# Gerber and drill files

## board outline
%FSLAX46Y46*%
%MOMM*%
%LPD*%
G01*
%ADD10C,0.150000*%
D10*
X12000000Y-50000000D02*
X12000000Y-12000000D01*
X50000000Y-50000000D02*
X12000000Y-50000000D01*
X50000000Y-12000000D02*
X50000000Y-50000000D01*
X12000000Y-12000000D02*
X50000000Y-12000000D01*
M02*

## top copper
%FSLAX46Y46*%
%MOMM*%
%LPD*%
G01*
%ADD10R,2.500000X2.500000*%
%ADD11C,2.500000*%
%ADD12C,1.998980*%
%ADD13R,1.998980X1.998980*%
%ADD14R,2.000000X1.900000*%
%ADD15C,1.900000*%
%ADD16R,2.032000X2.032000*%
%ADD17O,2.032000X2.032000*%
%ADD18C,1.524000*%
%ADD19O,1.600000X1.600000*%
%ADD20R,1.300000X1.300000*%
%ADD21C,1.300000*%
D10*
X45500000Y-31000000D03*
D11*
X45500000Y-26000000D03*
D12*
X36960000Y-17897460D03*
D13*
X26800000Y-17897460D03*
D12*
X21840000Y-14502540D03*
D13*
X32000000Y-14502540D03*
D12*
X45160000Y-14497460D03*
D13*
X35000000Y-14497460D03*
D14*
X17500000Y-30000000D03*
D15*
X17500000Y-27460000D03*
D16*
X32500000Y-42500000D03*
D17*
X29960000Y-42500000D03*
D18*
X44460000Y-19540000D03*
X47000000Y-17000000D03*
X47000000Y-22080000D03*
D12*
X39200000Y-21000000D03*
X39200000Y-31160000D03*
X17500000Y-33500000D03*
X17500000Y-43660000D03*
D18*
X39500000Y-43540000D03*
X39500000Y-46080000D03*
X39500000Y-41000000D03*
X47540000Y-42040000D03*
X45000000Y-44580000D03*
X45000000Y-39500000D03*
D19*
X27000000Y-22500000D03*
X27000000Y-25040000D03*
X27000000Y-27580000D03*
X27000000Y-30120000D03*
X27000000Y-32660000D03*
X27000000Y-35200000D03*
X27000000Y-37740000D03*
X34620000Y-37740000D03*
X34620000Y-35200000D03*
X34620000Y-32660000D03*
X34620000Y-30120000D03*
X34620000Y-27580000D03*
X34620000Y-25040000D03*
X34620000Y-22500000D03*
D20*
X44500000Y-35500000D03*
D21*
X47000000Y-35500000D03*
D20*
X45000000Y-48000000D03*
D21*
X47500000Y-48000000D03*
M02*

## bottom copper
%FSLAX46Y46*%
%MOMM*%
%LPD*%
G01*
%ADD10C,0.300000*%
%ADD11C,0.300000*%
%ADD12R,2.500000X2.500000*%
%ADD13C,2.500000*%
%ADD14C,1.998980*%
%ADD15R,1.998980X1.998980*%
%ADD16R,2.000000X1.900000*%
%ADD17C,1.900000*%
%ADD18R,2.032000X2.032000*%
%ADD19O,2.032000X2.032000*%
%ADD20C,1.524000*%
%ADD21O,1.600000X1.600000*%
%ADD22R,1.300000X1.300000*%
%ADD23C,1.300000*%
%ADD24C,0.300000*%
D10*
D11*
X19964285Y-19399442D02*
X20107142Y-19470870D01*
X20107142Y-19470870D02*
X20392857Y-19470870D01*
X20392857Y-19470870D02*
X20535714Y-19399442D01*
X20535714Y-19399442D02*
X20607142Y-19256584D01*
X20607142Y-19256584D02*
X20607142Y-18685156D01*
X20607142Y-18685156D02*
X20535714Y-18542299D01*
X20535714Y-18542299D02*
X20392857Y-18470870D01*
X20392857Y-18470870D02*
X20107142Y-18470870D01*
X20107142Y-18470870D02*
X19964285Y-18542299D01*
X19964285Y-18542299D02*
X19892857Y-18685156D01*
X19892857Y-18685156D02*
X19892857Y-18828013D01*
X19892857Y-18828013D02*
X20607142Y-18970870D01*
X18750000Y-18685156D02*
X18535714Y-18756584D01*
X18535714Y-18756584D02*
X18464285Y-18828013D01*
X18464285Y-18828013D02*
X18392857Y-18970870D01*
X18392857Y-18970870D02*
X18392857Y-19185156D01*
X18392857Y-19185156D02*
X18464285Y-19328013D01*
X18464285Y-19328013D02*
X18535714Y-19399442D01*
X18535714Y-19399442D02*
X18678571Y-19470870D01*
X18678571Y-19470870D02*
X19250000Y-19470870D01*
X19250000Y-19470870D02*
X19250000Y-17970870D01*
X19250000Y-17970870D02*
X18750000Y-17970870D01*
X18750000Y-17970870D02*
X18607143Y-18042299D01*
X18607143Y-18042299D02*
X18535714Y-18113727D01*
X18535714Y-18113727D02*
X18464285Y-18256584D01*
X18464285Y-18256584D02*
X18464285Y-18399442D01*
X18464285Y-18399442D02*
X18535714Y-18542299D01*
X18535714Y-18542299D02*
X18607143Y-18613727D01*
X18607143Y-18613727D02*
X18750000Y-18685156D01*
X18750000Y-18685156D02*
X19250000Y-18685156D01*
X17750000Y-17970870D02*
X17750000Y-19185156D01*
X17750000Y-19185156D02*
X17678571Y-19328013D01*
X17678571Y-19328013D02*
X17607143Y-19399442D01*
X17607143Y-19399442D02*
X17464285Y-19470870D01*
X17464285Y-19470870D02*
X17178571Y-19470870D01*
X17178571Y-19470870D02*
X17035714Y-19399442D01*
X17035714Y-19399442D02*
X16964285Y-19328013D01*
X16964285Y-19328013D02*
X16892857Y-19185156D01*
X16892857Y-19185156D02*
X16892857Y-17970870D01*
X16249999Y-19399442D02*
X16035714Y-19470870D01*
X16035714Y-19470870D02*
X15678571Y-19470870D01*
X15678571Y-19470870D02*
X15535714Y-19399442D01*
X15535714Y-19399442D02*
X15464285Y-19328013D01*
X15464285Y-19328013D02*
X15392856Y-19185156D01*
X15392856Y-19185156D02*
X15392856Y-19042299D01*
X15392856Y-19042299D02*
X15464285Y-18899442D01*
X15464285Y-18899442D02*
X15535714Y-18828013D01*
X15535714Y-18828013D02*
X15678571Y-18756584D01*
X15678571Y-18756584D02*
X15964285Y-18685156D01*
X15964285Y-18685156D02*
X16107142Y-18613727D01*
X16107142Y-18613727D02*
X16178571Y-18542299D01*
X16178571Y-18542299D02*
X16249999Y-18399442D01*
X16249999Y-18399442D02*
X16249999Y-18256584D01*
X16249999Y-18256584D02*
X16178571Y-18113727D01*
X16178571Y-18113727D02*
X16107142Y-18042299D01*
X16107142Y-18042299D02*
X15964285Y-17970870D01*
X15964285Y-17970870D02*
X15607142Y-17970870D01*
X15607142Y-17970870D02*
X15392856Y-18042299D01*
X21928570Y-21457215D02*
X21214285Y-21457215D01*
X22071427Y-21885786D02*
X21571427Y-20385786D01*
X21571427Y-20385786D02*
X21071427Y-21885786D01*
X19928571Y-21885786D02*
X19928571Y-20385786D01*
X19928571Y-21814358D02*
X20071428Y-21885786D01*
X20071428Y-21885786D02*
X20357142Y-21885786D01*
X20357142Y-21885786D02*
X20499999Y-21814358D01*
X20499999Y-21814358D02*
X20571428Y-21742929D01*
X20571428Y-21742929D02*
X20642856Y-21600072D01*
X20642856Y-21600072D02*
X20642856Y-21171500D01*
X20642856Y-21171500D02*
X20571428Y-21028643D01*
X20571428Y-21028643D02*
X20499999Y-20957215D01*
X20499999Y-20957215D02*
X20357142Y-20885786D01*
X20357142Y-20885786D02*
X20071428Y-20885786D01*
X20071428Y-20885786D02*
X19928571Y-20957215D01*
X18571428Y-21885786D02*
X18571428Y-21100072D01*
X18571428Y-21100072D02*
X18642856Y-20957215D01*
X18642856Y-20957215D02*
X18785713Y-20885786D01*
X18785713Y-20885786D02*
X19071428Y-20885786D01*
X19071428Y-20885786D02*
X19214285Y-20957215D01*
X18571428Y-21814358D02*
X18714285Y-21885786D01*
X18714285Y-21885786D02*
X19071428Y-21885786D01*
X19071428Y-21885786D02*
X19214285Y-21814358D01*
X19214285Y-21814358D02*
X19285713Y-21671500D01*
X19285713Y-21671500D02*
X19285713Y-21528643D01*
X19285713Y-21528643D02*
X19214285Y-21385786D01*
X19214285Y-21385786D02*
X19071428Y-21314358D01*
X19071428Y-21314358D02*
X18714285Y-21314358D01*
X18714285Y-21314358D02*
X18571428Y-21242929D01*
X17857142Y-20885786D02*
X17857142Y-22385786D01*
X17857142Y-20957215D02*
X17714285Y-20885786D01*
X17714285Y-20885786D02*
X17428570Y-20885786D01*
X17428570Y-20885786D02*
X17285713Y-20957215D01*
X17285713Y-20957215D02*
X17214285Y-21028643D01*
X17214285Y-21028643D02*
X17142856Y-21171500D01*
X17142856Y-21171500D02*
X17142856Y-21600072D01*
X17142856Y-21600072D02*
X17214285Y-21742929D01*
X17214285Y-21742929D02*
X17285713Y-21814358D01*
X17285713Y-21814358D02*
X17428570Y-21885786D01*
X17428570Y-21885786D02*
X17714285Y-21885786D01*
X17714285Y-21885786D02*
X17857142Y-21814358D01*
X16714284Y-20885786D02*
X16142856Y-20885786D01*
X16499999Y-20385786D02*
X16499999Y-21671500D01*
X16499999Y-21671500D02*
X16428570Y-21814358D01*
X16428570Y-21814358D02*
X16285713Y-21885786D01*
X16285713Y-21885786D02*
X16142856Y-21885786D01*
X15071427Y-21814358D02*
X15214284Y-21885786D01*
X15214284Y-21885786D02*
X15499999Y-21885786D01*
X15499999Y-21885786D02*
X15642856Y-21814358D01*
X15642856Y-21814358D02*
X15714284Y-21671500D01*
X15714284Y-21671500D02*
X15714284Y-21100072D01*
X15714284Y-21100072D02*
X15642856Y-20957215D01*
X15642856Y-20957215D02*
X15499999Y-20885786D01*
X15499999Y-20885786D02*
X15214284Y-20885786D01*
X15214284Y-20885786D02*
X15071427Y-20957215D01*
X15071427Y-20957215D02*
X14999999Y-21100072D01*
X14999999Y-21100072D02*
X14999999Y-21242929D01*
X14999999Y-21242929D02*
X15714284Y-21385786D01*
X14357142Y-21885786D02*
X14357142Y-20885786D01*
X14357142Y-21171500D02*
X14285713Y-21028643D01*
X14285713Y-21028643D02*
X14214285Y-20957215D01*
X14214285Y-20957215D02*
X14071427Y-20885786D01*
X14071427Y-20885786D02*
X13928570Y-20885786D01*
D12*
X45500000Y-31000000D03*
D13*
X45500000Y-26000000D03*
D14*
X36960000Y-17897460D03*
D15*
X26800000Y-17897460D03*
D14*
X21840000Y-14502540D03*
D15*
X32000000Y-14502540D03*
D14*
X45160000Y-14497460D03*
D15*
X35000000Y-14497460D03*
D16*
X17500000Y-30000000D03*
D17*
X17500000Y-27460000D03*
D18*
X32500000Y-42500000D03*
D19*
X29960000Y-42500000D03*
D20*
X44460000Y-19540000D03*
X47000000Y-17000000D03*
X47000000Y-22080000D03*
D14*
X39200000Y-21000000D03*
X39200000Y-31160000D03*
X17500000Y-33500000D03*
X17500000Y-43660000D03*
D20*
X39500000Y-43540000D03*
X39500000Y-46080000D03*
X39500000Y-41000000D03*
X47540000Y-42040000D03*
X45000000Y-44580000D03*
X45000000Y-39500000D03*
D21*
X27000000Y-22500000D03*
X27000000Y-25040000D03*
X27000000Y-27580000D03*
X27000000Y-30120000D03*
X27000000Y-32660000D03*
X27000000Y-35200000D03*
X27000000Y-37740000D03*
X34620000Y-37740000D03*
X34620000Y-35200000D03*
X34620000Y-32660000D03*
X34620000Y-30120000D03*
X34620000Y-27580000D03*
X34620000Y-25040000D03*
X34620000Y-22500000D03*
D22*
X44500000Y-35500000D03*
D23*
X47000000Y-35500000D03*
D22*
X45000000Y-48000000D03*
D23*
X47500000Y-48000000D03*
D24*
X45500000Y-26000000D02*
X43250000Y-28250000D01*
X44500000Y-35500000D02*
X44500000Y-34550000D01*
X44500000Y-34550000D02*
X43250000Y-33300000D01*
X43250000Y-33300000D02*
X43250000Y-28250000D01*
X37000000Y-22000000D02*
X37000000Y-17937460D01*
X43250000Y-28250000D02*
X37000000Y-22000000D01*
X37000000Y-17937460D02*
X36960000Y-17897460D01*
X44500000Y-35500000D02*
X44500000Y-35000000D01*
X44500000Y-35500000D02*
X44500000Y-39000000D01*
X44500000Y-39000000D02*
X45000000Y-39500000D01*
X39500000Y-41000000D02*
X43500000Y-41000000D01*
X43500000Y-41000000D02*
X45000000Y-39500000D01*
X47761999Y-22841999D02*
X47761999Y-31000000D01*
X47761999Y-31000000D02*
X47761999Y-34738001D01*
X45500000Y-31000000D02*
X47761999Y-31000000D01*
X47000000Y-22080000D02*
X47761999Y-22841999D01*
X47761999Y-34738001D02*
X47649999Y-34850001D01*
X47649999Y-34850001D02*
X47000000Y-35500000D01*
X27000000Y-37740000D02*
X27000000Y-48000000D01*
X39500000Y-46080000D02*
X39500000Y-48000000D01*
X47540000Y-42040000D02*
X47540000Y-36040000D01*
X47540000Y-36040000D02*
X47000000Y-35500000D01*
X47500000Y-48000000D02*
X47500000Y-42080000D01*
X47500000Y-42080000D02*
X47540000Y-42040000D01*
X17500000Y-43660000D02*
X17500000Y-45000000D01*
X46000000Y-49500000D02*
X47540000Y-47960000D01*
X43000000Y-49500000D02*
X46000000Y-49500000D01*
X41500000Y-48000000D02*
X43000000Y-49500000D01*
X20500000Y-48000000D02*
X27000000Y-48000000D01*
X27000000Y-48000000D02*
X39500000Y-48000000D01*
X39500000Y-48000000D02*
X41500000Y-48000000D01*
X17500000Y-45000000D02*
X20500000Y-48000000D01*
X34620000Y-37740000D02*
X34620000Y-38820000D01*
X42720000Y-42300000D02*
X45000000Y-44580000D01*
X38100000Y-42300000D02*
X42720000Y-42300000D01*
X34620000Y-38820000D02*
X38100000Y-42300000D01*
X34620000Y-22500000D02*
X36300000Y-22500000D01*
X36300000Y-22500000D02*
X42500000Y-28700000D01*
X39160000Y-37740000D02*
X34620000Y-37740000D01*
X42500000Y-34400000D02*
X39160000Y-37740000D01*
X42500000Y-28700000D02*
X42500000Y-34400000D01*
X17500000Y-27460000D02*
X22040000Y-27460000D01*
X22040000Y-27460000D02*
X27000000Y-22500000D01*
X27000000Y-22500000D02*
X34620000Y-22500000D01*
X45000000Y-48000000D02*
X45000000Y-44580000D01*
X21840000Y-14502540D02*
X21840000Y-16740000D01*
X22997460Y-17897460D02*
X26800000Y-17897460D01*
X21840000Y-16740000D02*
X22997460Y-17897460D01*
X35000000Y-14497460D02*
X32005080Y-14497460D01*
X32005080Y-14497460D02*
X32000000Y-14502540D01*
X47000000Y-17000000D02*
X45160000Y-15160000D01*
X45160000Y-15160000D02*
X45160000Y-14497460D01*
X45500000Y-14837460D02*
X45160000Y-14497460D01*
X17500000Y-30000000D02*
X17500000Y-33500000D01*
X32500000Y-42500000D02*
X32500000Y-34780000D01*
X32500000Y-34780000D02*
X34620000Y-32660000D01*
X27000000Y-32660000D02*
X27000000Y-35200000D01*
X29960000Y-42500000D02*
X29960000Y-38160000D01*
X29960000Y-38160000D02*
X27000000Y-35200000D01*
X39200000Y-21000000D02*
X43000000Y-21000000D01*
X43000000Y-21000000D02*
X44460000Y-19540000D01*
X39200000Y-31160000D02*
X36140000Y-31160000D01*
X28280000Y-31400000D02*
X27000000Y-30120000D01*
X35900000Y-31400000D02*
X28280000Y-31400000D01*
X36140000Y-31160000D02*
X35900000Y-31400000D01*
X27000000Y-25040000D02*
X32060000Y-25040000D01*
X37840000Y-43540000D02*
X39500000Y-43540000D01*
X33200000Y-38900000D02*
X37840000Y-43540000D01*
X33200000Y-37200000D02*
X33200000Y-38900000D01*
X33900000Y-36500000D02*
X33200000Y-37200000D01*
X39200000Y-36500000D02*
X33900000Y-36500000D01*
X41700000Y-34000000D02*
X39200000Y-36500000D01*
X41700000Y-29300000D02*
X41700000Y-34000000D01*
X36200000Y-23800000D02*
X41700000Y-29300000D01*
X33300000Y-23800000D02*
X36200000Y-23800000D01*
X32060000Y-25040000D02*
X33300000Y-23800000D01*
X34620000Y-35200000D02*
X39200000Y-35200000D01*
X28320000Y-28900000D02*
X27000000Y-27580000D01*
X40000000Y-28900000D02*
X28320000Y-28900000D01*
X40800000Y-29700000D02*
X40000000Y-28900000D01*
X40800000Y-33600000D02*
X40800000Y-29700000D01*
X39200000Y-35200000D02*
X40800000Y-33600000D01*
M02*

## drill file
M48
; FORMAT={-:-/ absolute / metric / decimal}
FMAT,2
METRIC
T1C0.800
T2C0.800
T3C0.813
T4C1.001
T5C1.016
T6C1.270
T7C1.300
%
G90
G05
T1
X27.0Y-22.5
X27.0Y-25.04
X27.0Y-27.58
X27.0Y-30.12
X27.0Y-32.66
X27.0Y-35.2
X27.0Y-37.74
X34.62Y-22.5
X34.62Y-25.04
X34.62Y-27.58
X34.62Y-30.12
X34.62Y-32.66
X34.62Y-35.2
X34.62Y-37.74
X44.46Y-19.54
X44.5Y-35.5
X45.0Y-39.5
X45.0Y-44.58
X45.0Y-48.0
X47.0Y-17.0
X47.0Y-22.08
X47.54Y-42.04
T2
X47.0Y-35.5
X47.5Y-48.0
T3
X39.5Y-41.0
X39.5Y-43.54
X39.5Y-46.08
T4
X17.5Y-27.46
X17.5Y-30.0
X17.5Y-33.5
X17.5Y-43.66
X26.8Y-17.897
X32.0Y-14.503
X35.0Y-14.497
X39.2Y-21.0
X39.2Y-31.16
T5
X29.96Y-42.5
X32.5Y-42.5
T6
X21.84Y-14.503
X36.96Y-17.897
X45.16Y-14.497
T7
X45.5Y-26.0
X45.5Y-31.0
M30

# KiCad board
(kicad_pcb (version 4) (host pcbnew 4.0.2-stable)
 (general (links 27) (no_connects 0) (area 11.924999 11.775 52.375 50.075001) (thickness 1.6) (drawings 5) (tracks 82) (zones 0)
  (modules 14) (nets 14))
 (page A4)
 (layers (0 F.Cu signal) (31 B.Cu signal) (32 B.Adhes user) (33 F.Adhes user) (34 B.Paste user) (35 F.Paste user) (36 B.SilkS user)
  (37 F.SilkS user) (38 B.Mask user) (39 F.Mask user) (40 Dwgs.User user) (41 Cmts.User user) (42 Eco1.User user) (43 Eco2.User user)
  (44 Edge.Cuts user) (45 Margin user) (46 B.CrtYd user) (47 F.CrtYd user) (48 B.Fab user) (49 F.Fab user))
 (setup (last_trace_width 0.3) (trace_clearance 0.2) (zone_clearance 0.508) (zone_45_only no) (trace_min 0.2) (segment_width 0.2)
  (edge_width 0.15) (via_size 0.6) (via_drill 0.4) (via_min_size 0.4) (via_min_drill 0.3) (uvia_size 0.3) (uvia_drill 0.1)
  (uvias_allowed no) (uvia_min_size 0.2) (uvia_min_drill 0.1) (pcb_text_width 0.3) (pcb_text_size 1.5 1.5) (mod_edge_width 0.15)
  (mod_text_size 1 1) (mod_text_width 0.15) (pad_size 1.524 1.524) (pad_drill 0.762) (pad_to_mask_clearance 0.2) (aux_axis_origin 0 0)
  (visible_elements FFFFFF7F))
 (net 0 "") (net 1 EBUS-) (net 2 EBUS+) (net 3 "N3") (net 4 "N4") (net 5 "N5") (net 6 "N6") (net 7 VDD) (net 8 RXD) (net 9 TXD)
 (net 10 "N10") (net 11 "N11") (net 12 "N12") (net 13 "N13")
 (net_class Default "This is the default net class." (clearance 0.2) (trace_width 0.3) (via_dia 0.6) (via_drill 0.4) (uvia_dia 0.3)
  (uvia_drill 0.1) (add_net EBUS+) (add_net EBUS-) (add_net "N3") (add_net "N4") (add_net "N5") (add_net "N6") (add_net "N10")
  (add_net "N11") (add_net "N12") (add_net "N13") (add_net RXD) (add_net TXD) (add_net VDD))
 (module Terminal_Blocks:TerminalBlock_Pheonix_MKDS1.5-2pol (layer F.Cu) (at 45.5 31 90)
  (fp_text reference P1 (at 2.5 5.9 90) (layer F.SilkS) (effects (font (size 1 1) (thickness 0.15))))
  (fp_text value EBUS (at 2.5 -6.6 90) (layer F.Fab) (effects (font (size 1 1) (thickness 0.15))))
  (pad 1 thru_hole rect (at 0 0 90) (size 2.5 2.5) (drill 1.3) (layers *.Cu *.Mask F.SilkS) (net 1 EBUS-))
  (pad 2 thru_hole circle (at 5 0 90) (size 2.5 2.5) (drill 1.3) (layers *.Cu *.Mask F.SilkS) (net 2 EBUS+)))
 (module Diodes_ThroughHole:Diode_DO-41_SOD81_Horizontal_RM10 (layer F.Cu) (at 26.8 17.9)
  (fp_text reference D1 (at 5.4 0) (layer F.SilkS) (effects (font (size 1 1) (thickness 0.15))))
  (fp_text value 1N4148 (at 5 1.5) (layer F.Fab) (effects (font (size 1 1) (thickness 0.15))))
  (pad 2 thru_hole circle (at 10.16 -0.00254 180) (size 1.99898 1.99898) (drill 1.27) (layers *.Cu *.Mask F.SilkS) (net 2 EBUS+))
  (pad 1 thru_hole rect (at 0 -0.00254 180) (size 1.99898 1.99898) (drill 1.00076) (layers *.Cu *.Mask F.SilkS) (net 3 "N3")))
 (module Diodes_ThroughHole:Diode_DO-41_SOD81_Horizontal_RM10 (layer F.Cu) (at 32 14.5 180)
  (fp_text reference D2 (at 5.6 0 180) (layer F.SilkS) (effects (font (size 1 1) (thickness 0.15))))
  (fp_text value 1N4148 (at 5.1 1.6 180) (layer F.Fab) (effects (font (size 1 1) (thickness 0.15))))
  (pad 2 thru_hole circle (at 10.16 -0.00254) (size 1.99898 1.99898) (drill 1.27) (layers *.Cu *.Mask F.SilkS) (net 3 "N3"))
  (pad 1 thru_hole rect (at 0 -0.00254) (size 1.99898 1.99898) (drill 1.00076) (layers *.Cu *.Mask F.SilkS) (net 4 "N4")))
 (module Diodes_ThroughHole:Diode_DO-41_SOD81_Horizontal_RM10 (layer F.Cu) (at 35 14.5)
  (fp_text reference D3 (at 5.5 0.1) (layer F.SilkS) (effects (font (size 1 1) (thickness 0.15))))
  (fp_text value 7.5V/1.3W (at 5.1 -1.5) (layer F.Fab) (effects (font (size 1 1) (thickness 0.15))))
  (pad 2 thru_hole circle (at 10.16 -0.00254 180) (size 1.99898 1.99898) (drill 1.27) (layers *.Cu *.Mask F.SilkS) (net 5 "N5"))
  (pad 1 thru_hole rect (at 0 -0.00254 180) (size 1.99898 1.99898) (drill 1.00076) (layers *.Cu *.Mask F.SilkS) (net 4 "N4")))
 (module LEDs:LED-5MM (layer F.Cu) (at 17.5 30 90)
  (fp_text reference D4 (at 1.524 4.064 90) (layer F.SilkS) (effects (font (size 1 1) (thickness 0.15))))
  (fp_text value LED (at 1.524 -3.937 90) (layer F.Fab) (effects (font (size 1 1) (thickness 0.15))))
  (pad 1 thru_hole rect (at 0 0 180) (size 2 1.9) (drill 1.00076) (layers *.Cu *.Mask F.SilkS) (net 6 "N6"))
  (pad 2 thru_hole circle (at 2.54 0 90) (size 1.9 1.9) (drill 1.00076) (layers *.Cu *.Mask F.SilkS) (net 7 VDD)))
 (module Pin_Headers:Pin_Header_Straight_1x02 (layer F.Cu) (at 32.5 42.5 270)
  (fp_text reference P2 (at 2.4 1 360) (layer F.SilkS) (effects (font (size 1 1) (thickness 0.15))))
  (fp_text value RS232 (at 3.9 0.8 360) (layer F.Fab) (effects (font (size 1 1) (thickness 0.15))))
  (pad 1 thru_hole rect (at 0 0 270) (size 2.032 2.032) (drill 1.016) (layers *.Cu *.Mask F.SilkS) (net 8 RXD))
  (pad 2 thru_hole oval (at 0 2.54 270) (size 2.032 2.032) (drill 1.016) (layers *.Cu *.Mask F.SilkS) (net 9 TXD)))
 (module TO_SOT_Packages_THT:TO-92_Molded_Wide (layer F.Cu) (at 47 22.08 90)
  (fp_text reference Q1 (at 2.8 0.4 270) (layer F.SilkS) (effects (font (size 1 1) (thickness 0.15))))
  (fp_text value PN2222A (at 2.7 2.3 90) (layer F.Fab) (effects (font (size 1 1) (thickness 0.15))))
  (pad 2 thru_hole circle (at 2.54 -2.54 180) (size 1.524 1.524) (drill 0.8) (layers *.Cu *.Mask F.SilkS) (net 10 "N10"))
  (pad 3 thru_hole circle (at 5.08 0 180) (size 1.524 1.524) (drill 0.8) (layers *.Cu *.Mask F.SilkS) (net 5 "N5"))
  (pad 1 thru_hole circle (at 0 0 180) (size 1.524 1.524) (drill 0.8) (layers *.Cu *.Mask F.SilkS) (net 1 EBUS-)))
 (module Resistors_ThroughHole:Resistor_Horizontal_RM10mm (layer F.Cu) (at 39.2 21 270)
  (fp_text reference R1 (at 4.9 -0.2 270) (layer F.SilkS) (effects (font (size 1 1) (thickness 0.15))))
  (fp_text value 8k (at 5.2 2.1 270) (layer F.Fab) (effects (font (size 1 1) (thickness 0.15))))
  (pad 1 thru_hole circle (at 0 0 270) (size 1.99898 1.99898) (drill 1.00076) (layers *.Cu *.SilkS *.Mask) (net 10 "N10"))
  (pad 2 thru_hole circle (at 10.16 0 270) (size 1.99898 1.99898) (drill 1.00076) (layers *.Cu *.SilkS *.Mask) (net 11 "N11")))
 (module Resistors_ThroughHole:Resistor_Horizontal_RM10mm (layer F.Cu) (at 17.5 33.5 270)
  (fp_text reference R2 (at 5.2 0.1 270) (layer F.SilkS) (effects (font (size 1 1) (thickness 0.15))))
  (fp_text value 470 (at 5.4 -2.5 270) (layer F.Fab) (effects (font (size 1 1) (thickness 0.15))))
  (pad 1 thru_hole circle (at 0 0 270) (size 1.99898 1.99898) (drill 1.00076) (layers *.Cu *.SilkS *.Mask) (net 6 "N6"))
  (pad 2 thru_hole circle (at 10.16 0 270) (size 1.99898 1.99898) (drill 1.00076) (layers *.Cu *.SilkS *.Mask) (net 1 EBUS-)))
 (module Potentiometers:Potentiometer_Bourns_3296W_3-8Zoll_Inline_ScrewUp (layer F.Cu) (at 39.5 41 180)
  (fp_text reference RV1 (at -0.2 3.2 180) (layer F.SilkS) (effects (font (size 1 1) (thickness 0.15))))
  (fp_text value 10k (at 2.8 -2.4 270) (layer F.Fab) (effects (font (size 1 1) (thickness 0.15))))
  (pad 2 thru_hole circle (at 0 -2.54 180) (size 1.524 1.524) (drill 0.8128) (layers *.Cu *.Mask F.SilkS) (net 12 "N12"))
  (pad 3 thru_hole circle (at 0 -5.08 180) (size 1.524 1.524) (drill 0.8128) (layers *.Cu *.Mask F.SilkS) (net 1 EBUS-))
  (pad 1 thru_hole circle (at 0 0 180) (size 1.524 1.524) (drill 0.8128) (layers *.Cu *.Mask F.SilkS) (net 2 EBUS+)))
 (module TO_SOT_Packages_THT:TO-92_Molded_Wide (layer F.Cu) (at 45 39.5 270)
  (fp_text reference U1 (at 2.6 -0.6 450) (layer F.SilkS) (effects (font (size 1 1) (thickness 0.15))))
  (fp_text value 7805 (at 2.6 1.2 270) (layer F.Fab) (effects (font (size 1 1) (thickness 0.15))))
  (pad 2 thru_hole circle (at 2.54 -2.54) (size 1.524 1.524) (drill 0.8) (layers *.Cu *.Mask F.SilkS) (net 1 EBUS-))
  (pad 3 thru_hole circle (at 5.08 0) (size 1.524 1.524) (drill 0.8) (layers *.Cu *.Mask F.SilkS) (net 7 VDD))
  (pad 1 thru_hole circle (at 0 0) (size 1.524 1.524) (drill 0.8) (layers *.Cu *.Mask F.SilkS) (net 2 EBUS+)))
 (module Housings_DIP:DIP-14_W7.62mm (layer F.Cu) (at 27 22.5)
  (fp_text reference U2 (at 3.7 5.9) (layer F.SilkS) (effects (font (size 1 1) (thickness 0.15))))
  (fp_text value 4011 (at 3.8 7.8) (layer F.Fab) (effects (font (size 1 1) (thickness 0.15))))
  (pad 1 thru_hole oval (at 0 0) (size 1.6 1.6) (drill 0.8) (layers *.Cu *.Mask F.SilkS) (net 7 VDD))
  (pad 2 thru_hole oval (at 0 2.54) (size 1.6 1.6) (drill 0.8) (layers *.Cu *.Mask F.SilkS) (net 12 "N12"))
  (pad 3 thru_hole oval (at 0 5.08) (size 1.6 1.6) (drill 0.8) (layers *.Cu *.Mask F.SilkS) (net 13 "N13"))
  (pad 4 thru_hole oval (at 0 7.62) (size 1.6 1.6) (drill 0.8) (layers *.Cu *.Mask F.SilkS) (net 11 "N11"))
  (pad 5 thru_hole oval (at 0 10.16) (size 1.6 1.6) (drill 0.8) (layers *.Cu *.Mask F.SilkS) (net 9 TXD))
  (pad 6 thru_hole oval (at 0 12.7) (size 1.6 1.6) (drill 0.8) (layers *.Cu *.Mask F.SilkS) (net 9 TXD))
  (pad 7 thru_hole oval (at 0 15.24) (size 1.6 1.6) (drill 0.8) (layers *.Cu *.Mask F.SilkS) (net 1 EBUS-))
  (pad 8 thru_hole oval (at 7.62 15.24) (size 1.6 1.6) (drill 0.8) (layers *.Cu *.Mask F.SilkS) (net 7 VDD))
  (pad 9 thru_hole oval (at 7.62 12.7) (size 1.6 1.6) (drill 0.8) (layers *.Cu *.Mask F.SilkS) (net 13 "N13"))
  (pad 10 thru_hole oval (at 7.62 10.16) (size 1.6 1.6) (drill 0.8) (layers *.Cu *.Mask F.SilkS) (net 8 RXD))
  (pad 11 thru_hole oval (at 7.62 7.62) (size 1.6 1.6) (drill 0.8) (layers *.Cu *.Mask F.SilkS))
  (pad 12 thru_hole oval (at 7.62 5.08) (size 1.6 1.6) (drill 0.8) (layers *.Cu *.Mask F.SilkS))
  (pad 13 thru_hole oval (at 7.62 2.54) (size 1.6 1.6) (drill 0.8) (layers *.Cu *.Mask F.SilkS))
  (pad 14 thru_hole oval (at 7.62 0) (size 1.6 1.6) (drill 0.8) (layers *.Cu *.Mask F.SilkS) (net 7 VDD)))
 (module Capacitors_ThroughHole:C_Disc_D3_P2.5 (layer F.Cu) (at 44.5 35.5)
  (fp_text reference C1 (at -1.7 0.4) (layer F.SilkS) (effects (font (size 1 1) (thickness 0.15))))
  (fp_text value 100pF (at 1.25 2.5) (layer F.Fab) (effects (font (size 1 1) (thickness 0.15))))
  (pad 1 thru_hole rect (at 0 0) (size 1.3 1.3) (drill 0.8) (layers *.Cu *.Mask F.SilkS) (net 2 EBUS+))
  (pad 2 thru_hole circle (at 2.5 0) (size 1.3 1.3) (drill 0.8001) (layers *.Cu *.Mask F.SilkS) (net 1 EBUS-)))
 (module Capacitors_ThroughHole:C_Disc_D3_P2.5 (layer F.Cu) (at 45 48)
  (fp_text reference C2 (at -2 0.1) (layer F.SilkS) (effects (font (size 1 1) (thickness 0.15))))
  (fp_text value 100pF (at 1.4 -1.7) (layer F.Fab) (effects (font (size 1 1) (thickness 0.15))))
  (pad 1 thru_hole rect (at 0 0) (size 1.3 1.3) (drill 0.8) (layers *.Cu *.Mask F.SilkS) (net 7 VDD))
  (pad 2 thru_hole circle (at 2.5 0) (size 1.3 1.3) (drill 0.8001) (layers *.Cu *.Mask F.SilkS) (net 1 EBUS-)))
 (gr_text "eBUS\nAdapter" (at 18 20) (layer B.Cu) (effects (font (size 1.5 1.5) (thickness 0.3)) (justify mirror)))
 (gr_line (start 12 50) (end 12 12) (angle 90) (layer Edge.Cuts) (width 0.15))
 (gr_line (start 50 50) (end 12 50) (angle 90) (layer Edge.Cuts) (width 0.15))
 (gr_line (start 50 12) (end 50 50) (angle 90) (layer Edge.Cuts) (width 0.15))
 (gr_line (start 12 12) (end 50 12) (angle 90) (layer Edge.Cuts) (width 0.15))
 (segment (start 45.5 26) (end 43.25 28.25) (width 0.3) (layer B.Cu) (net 2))
 (segment (start 44.5 35.5) (end 44.5 34.55) (width 0.3) (layer B.Cu) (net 2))
 (segment (start 44.5 34.55) (end 43.25 33.3) (width 0.3) (layer B.Cu) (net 2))
 (segment (start 43.25 33.3) (end 43.25 28.25) (width 0.3) (layer B.Cu) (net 2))
 (segment (start 37 22) (end 37 17.93746) (width 0.3) (layer B.Cu) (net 2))
 (segment (start 43.25 28.25) (end 37 22) (width 0.3) (layer B.Cu) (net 2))
 (segment (start 37 17.93746) (end 36.96 17.89746) (width 0.3) (layer B.Cu) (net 2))
 (segment (start 44.5 35.5) (end 44.5 35) (width 0.3) (layer B.Cu) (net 2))
 (segment (start 44.5 35.5) (end 44.5 39) (width 0.3) (layer B.Cu) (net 2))
 (segment (start 44.5 39) (end 45 39.5) (width 0.3) (layer B.Cu) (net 2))
 (segment (start 39.5 41) (end 43.5 41) (width 0.3) (layer B.Cu) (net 2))
 (segment (start 43.5 41) (end 45 39.5) (width 0.3) (layer B.Cu) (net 2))
 (segment (start 47.761999 22.841999) (end 47.761999 31) (width 0.3) (layer B.Cu) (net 1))
 (segment (start 47.761999 31) (end 47.761999 34.738001) (width 0.3) (layer B.Cu) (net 1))
 (segment (start 45.5 31) (end 47.761999 31) (width 0.3) (layer B.Cu) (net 1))
 (segment (start 47 22.08) (end 47.761999 22.841999) (width 0.3) (layer B.Cu) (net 1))
 (segment (start 47.761999 34.738001) (end 47.649999 34.850001) (width 0.3) (layer B.Cu) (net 1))
 (segment (start 47.649999 34.850001) (end 47 35.5) (width 0.3) (layer B.Cu) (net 1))
 (segment (start 27 37.74) (end 27 48) (width 0.3) (layer B.Cu) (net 1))
 (segment (start 39.5 46.08) (end 39.5 48) (width 0.3) (layer B.Cu) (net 1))
 (segment (start 47.54 42.04) (end 47.54 36.04) (width 0.3) (layer B.Cu) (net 1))
 (segment (start 47.54 36.04) (end 47 35.5) (width 0.3) (layer B.Cu) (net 1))
 (segment (start 47.5 48) (end 47.5 42.08) (width 0.3) (layer B.Cu) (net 1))
 (segment (start 47.5 42.08) (end 47.54 42.04) (width 0.3) (layer B.Cu) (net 1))
 (segment (start 17.5 43.66) (end 17.5 45) (width 0.3) (layer B.Cu) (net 1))
 (segment (start 46 49.5) (end 47.54 47.96) (width 0.3) (layer B.Cu) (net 1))
 (segment (start 43 49.5) (end 46 49.5) (width 0.3) (layer B.Cu) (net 1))
 (segment (start 41.5 48) (end 43 49.5) (width 0.3) (layer B.Cu) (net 1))
 (segment (start 20.5 48) (end 27 48) (width 0.3) (layer B.Cu) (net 1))
 (segment (start 27 48) (end 39.5 48) (width 0.3) (layer B.Cu) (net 1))
 (segment (start 39.5 48) (end 41.5 48) (width 0.3) (layer B.Cu) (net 1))
 (segment (start 17.5 45) (end 20.5 48) (width 0.3) (layer B.Cu) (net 1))
 (segment (start 34.62 37.74) (end 34.62 38.82) (width 0.3) (layer B.Cu) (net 7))
 (segment (start 42.72 42.3) (end 45 44.58) (width 0.3) (layer B.Cu) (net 7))
 (segment (start 38.1 42.3) (end 42.72 42.3) (width 0.3) (layer B.Cu) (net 7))
 (segment (start 34.62 38.82) (end 38.1 42.3) (width 0.3) (layer B.Cu) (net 7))
 (segment (start 34.62 22.5) (end 36.3 22.5) (width 0.3) (layer B.Cu) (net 7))
 (segment (start 36.3 22.5) (end 42.5 28.7) (width 0.3) (layer B.Cu) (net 7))
 (segment (start 39.16 37.74) (end 34.62 37.74) (width 0.3) (layer B.Cu) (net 7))
 (segment (start 42.5 34.4) (end 39.16 37.74) (width 0.3) (layer B.Cu) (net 7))
 (segment (start 42.5 28.7) (end 42.5 34.4) (width 0.3) (layer B.Cu) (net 7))
 (segment (start 17.5 27.46) (end 22.04 27.46) (width 0.3) (layer B.Cu) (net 7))
 (segment (start 22.04 27.46) (end 27 22.5) (width 0.3) (layer B.Cu) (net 7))
 (segment (start 27 22.5) (end 34.62 22.5) (width 0.3) (layer B.Cu) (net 7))
 (segment (start 45 48) (end 45 44.58) (width 0.3) (layer B.Cu) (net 7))
 (segment (start 21.84 14.50254) (end 21.84 16.74) (width 0.3) (layer B.Cu) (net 3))
 (segment (start 22.99746 17.89746) (end 26.8 17.89746) (width 0.3) (layer B.Cu) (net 3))
 (segment (start 21.84 16.74) (end 22.99746 17.89746) (width 0.3) (layer B.Cu) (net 3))
 (segment (start 35 14.49746) (end 32.00508 14.49746) (width 0.3) (layer B.Cu) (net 4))
 (segment (start 32.00508 14.49746) (end 32 14.50254) (width 0.3) (layer B.Cu) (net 4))
 (segment (start 47 17) (end 45.16 15.16) (width 0.3) (layer B.Cu) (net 5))
 (segment (start 45.16 15.16) (end 45.16 14.49746) (width 0.3) (layer B.Cu) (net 5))
 (segment (start 45.5 14.83746) (end 45.16 14.49746) (width 0.3) (layer B.Cu) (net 5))
 (segment (start 17.5 30) (end 17.5 33.5) (width 0.3) (layer B.Cu) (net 6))
 (segment (start 32.5 42.5) (end 32.5 34.78) (width 0.3) (layer B.Cu) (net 8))
 (segment (start 32.5 34.78) (end 34.62 32.66) (width 0.3) (layer B.Cu) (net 8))
 (segment (start 27 32.66) (end 27 35.2) (width 0.3) (layer B.Cu) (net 9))
 (segment (start 29.96 42.5) (end 29.96 38.16) (width 0.3) (layer B.Cu) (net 9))
 (segment (start 29.96 38.16) (end 27 35.2) (width 0.3) (layer B.Cu) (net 9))
 (segment (start 39.2 21) (end 43 21) (width 0.3) (layer B.Cu) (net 10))
 (segment (start 43 21) (end 44.46 19.54) (width 0.3) (layer B.Cu) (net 10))
 (segment (start 39.2 31.16) (end 36.14 31.16) (width 0.3) (layer B.Cu) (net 11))
 (segment (start 28.28 31.4) (end 27 30.12) (width 0.3) (layer B.Cu) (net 11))
 (segment (start 35.9 31.4) (end 28.28 31.4) (width 0.3) (layer B.Cu) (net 11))
 (segment (start 36.14 31.16) (end 35.9 31.4) (width 0.3) (layer B.Cu) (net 11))
 (segment (start 27 25.04) (end 32.06 25.04) (width 0.3) (layer B.Cu) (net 12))
 (segment (start 37.84 43.54) (end 39.5 43.54) (width 0.3) (layer B.Cu) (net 12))
 (segment (start 33.2 38.9) (end 37.84 43.54) (width 0.3) (layer B.Cu) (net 12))
 (segment (start 33.2 37.2) (end 33.2 38.9) (width 0.3) (layer B.Cu) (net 12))
 (segment (start 33.9 36.5) (end 33.2 37.2) (width 0.3) (layer B.Cu) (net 12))
 (segment (start 39.2 36.5) (end 33.9 36.5) (width 0.3) (layer B.Cu) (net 12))
 (segment (start 41.7 34) (end 39.2 36.5) (width 0.3) (layer B.Cu) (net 12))
 (segment (start 41.7 29.3) (end 41.7 34) (width 0.3) (layer B.Cu) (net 12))
 (segment (start 36.2 23.8) (end 41.7 29.3) (width 0.3) (layer B.Cu) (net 12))
 (segment (start 33.3 23.8) (end 36.2 23.8) (width 0.3) (layer B.Cu) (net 12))
 (segment (start 32.06 25.04) (end 33.3 23.8) (width 0.3) (layer B.Cu) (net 12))
 (segment (start 34.62 35.2) (end 39.2 35.2) (width 0.3) (layer B.Cu) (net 13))
 (segment (start 28.32 28.9) (end 27 27.58) (width 0.3) (layer B.Cu) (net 13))
 (segment (start 40 28.9) (end 28.32 28.9) (width 0.3) (layer B.Cu) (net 13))
 (segment (start 40.8 29.7) (end 40 28.9) (width 0.3) (layer B.Cu) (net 13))
 (segment (start 40.8 33.6) (end 40.8 29.7) (width 0.3) (layer B.Cu) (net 13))
 (segment (start 39.2 35.2) (end 40.8 33.6) (width 0.3) (layer B.Cu) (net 13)))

